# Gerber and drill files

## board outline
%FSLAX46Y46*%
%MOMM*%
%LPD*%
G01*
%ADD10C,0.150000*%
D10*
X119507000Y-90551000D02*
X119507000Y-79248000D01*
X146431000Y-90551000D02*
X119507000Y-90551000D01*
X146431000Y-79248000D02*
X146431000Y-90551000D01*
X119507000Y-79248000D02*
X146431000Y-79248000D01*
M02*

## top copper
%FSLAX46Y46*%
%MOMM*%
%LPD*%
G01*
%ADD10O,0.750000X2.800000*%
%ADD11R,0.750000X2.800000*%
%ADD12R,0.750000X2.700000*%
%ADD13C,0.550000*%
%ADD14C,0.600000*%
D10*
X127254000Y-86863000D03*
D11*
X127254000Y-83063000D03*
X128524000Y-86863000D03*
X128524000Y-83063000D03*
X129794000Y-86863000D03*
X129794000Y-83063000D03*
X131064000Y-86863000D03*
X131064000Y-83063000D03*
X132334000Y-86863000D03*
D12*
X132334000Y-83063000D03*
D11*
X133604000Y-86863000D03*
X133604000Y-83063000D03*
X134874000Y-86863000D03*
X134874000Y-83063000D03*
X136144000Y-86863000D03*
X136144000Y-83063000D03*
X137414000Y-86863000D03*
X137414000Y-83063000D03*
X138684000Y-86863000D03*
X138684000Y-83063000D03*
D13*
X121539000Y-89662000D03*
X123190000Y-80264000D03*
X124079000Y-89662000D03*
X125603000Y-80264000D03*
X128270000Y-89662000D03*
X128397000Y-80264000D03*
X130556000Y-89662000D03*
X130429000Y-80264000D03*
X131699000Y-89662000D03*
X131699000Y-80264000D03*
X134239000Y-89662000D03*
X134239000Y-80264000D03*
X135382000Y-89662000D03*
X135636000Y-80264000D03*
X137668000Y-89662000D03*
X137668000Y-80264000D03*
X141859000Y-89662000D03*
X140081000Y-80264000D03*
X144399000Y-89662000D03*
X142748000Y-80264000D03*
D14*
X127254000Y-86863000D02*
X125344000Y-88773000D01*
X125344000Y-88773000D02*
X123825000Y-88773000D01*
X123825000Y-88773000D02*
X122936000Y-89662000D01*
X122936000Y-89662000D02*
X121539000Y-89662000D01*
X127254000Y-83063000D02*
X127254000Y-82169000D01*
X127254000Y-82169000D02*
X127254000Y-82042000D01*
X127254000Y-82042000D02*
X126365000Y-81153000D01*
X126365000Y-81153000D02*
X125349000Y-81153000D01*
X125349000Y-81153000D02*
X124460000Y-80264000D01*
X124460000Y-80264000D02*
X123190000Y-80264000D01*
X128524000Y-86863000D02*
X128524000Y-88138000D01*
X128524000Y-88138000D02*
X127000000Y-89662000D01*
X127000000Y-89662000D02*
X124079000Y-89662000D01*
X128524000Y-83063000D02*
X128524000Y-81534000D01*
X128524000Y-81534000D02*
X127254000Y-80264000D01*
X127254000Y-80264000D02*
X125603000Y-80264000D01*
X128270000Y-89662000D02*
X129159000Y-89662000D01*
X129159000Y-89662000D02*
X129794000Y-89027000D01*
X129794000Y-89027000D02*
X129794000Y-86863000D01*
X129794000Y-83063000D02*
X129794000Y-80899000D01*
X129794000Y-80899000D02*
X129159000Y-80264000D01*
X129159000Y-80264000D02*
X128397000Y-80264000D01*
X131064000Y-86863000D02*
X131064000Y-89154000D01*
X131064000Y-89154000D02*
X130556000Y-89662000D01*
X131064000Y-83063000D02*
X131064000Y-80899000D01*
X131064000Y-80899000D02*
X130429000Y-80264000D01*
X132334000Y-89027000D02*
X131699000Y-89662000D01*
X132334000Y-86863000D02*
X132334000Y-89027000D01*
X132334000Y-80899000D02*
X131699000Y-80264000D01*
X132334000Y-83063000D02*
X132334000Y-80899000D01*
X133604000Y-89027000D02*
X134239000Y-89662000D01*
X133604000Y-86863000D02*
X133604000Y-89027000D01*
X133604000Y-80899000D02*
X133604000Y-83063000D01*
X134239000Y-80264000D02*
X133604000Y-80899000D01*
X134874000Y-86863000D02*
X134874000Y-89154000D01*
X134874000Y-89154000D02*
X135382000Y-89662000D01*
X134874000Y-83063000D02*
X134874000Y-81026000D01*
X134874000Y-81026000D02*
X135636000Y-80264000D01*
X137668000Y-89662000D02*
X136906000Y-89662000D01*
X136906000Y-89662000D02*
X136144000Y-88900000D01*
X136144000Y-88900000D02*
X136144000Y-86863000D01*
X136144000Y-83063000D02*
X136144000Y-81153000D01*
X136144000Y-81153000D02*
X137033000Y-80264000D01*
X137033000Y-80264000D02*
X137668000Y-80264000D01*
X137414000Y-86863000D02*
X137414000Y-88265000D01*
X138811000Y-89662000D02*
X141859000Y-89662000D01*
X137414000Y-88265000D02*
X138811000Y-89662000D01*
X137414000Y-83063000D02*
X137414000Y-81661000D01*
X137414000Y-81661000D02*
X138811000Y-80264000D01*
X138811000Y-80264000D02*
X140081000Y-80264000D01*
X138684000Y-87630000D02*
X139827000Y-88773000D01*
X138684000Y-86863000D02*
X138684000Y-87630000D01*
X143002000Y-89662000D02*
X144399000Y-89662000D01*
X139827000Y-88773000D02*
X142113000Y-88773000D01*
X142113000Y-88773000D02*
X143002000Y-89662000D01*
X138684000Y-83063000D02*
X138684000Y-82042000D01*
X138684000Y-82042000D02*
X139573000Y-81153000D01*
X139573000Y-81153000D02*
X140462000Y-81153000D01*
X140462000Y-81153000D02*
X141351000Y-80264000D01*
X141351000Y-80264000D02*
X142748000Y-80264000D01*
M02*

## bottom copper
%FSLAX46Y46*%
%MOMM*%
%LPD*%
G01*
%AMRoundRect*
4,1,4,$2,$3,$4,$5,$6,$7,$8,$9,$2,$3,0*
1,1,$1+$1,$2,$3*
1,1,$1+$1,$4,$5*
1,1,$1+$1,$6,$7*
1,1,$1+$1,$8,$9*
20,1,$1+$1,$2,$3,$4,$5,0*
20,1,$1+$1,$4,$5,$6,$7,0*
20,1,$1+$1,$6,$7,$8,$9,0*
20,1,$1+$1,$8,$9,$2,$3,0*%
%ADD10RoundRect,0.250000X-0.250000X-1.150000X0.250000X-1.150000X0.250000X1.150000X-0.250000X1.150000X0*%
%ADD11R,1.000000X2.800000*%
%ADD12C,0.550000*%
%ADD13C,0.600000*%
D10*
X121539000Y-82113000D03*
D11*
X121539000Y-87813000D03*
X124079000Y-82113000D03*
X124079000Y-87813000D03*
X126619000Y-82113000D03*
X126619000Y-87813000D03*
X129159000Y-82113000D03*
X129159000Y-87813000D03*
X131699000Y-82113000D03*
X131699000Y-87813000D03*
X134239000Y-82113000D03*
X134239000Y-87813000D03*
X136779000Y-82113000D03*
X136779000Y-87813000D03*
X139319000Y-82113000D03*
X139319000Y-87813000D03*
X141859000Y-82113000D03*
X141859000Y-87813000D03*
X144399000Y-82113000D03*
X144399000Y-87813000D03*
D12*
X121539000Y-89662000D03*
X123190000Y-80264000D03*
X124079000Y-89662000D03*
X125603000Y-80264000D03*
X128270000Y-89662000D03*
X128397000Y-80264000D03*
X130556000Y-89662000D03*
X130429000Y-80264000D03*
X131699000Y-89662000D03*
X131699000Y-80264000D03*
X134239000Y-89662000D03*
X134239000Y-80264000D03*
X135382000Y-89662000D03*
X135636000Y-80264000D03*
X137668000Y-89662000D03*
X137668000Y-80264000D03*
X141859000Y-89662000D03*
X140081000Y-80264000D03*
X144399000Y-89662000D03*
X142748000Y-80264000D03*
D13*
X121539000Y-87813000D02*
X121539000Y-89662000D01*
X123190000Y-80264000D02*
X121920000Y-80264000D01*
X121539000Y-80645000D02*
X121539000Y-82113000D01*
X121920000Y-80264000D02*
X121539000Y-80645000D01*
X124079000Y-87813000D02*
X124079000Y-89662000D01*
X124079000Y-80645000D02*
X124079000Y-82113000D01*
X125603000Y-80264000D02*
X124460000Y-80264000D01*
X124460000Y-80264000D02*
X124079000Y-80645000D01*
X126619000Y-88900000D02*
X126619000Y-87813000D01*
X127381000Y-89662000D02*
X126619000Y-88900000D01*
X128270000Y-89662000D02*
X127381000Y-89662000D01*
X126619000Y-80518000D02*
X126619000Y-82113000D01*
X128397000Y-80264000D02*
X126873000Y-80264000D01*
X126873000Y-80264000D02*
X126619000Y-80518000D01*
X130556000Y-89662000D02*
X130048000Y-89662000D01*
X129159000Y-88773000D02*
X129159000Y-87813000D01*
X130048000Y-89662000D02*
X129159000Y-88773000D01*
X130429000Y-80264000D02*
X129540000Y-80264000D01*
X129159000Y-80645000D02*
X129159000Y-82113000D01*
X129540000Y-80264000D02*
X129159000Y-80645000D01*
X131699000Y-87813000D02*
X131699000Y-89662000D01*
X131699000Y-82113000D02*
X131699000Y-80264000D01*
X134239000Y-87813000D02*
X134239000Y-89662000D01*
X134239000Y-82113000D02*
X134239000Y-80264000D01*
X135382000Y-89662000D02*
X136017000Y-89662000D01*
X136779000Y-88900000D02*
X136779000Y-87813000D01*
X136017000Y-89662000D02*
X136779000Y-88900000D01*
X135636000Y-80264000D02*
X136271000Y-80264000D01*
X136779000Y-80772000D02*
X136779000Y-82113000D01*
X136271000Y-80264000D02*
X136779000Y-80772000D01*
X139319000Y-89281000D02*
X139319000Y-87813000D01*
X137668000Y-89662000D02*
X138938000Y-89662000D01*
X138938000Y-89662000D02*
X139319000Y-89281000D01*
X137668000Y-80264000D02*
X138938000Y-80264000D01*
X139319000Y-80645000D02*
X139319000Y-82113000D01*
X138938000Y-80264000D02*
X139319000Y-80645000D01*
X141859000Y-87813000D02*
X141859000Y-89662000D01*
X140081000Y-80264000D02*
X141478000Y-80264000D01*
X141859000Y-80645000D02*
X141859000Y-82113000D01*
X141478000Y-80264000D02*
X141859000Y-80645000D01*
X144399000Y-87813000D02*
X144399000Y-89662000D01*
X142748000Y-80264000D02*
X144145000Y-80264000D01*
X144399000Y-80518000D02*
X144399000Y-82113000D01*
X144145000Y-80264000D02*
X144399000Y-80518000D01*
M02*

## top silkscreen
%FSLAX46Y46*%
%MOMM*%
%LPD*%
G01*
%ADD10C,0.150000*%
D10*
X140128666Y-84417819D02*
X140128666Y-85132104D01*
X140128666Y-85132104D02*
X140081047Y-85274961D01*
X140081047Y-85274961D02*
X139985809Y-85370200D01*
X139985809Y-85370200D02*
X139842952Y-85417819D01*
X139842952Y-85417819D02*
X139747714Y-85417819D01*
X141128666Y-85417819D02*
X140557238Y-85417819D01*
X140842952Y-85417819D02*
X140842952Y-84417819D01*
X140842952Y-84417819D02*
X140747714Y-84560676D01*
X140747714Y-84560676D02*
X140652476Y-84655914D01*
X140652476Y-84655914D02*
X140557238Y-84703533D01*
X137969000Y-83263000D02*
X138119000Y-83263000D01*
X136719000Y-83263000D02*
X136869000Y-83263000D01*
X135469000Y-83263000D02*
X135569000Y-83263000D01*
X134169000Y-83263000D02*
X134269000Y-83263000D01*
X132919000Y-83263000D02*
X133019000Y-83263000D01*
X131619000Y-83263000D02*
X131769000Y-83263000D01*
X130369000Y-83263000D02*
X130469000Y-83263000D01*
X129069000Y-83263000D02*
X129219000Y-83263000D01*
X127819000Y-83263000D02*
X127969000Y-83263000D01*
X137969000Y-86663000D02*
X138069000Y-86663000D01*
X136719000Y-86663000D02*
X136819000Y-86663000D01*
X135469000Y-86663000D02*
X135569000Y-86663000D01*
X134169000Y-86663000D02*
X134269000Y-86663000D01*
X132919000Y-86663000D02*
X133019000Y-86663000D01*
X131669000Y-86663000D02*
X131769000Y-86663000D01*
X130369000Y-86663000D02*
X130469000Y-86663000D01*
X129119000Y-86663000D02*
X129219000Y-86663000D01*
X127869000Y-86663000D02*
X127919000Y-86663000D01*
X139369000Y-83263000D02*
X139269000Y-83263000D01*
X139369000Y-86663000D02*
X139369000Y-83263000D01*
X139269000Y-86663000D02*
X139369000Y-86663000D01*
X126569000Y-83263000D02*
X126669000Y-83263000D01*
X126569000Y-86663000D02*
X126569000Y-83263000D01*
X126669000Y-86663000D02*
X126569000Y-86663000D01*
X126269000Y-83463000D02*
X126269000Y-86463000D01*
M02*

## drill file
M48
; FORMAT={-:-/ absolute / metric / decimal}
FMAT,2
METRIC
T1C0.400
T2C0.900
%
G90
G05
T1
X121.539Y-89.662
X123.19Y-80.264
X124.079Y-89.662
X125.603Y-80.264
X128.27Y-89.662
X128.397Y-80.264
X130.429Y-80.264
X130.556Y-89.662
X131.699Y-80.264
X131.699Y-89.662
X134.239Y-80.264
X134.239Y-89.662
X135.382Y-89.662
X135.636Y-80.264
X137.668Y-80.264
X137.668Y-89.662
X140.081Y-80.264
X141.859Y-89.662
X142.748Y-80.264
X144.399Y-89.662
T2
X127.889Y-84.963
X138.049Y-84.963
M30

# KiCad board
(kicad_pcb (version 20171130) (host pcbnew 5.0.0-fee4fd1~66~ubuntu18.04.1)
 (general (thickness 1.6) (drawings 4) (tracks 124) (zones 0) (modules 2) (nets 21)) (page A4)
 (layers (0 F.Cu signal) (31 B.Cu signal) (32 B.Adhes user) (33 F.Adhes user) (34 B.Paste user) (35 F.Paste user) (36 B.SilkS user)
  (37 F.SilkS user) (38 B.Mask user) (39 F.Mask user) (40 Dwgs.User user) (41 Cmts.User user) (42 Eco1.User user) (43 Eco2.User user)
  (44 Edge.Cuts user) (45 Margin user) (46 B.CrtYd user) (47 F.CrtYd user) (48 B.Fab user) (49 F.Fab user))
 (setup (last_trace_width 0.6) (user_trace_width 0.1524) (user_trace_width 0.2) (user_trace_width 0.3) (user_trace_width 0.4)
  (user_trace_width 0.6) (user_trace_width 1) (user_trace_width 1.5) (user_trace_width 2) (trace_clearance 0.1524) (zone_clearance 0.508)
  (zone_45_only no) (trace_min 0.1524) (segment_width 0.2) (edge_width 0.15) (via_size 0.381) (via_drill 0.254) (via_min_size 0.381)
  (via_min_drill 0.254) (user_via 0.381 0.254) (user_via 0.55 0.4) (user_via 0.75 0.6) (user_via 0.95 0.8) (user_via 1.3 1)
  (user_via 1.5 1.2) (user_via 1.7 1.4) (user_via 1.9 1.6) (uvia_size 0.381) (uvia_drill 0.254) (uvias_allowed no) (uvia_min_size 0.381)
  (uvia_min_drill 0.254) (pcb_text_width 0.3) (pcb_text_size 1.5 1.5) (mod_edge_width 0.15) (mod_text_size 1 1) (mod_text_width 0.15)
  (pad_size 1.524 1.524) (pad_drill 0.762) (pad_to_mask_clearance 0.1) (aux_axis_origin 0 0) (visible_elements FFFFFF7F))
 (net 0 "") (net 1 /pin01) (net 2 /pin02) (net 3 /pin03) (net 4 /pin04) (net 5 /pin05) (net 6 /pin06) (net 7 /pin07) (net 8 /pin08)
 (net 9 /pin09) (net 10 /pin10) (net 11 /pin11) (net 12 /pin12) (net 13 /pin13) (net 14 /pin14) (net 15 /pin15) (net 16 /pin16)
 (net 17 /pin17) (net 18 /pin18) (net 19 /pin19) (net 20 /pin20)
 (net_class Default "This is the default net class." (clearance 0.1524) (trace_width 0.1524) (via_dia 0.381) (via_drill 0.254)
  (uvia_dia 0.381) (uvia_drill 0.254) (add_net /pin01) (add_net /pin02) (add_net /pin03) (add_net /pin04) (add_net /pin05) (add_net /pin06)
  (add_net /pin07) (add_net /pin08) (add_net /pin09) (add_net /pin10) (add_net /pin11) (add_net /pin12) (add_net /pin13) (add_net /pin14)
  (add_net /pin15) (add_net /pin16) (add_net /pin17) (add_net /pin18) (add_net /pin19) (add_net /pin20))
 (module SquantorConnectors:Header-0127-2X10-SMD (layer F.Cu) (at 132.969 84.963)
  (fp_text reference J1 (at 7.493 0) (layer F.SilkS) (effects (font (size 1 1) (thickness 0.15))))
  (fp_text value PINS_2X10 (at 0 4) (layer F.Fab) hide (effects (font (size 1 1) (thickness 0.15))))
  (fp_line (start 5 -1.7) (end 5.15 -1.7) (layer F.SilkS) (width 0.15))
  (fp_line (start 3.75 -1.7) (end 3.9 -1.7) (layer F.SilkS) (width 0.15))
  (fp_line (start 2.5 -1.7) (end 2.6 -1.7) (layer F.SilkS) (width 0.15))
  (fp_line (start 1.2 -1.7) (end 1.3 -1.7) (layer F.SilkS) (width 0.15))
  (fp_line (start -0.05 -1.7) (end 0.05 -1.7) (layer F.SilkS) (width 0.15))
  (fp_line (start -1.35 -1.7) (end -1.2 -1.7) (layer F.SilkS) (width 0.15))
  (fp_line (start -2.6 -1.7) (end -2.5 -1.7) (layer F.SilkS) (width 0.15))
  (fp_line (start -3.9 -1.7) (end -3.75 -1.7) (layer F.SilkS) (width 0.15))
  (fp_line (start -5.15 -1.7) (end -5 -1.7) (layer F.SilkS) (width 0.15))
  (fp_line (start 5 1.7) (end 5.1 1.7) (layer F.SilkS) (width 0.15))
  (fp_line (start 3.75 1.7) (end 3.85 1.7) (layer F.SilkS) (width 0.15))
  (fp_line (start 2.5 1.7) (end 2.6 1.7) (layer F.SilkS) (width 0.15))
  (fp_line (start 1.2 1.7) (end 1.3 1.7) (layer F.SilkS) (width 0.15))
  (fp_line (start -0.05 1.7) (end 0.05 1.7) (layer F.SilkS) (width 0.15))
  (fp_line (start -1.3 1.7) (end -1.2 1.7) (layer F.SilkS) (width 0.15))
  (fp_line (start -2.6 1.7) (end -2.5 1.7) (layer F.SilkS) (width 0.15))
  (fp_line (start -3.85 1.7) (end -3.75 1.7) (layer F.SilkS) (width 0.15))
  (fp_line (start -5.1 1.7) (end -5.05 1.7) (layer F.SilkS) (width 0.15))
  (fp_line (start 6.4 -1.7) (end 6.3 -1.7) (layer F.SilkS) (width 0.15))
  (fp_line (start 6.4 1.7) (end 6.4 -1.7) (layer F.SilkS) (width 0.15))
  (fp_line (start 6.3 1.7) (end 6.4 1.7) (layer F.SilkS) (width 0.15))
  (fp_line (start -6.4 -1.7) (end -6.3 -1.7) (layer F.SilkS) (width 0.15))
  (fp_line (start -6.4 1.7) (end -6.4 -1.7) (layer F.SilkS) (width 0.15))
  (fp_line (start -6.3 1.7) (end -6.4 1.7) (layer F.SilkS) (width 0.15))
  (fp_line (start -6.7 -1.5) (end -6.7 1.5) (layer F.SilkS) (width 0.15))
  (pad 1 smd oval (at -5.715 1.9) (size 0.75 2.8) (layers F.Cu F.Paste F.Mask) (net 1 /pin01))
  (pad 2 smd rect (at -5.715 -1.9) (size 0.75 2.8) (layers F.Cu F.Paste F.Mask) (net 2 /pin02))
  (pad 3 smd rect (at -4.445 1.9) (size 0.75 2.8) (layers F.Cu F.Paste F.Mask) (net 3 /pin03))
  (pad 4 smd rect (at -4.445 -1.9) (size 0.75 2.8) (layers F.Cu F.Paste F.Mask) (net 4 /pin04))
  (pad 5 smd rect (at -3.175 1.9) (size 0.75 2.8) (layers F.Cu F.Paste F.Mask) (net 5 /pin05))
  (pad 6 smd rect (at -3.175 -1.9) (size 0.75 2.8) (layers F.Cu F.Paste F.Mask) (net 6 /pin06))
  (pad 7 smd rect (at -1.905 1.9) (size 0.75 2.8) (layers F.Cu F.Paste F.Mask) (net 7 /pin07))
  (pad 8 smd rect (at -1.905 -1.9) (size 0.75 2.8) (layers F.Cu F.Paste F.Mask) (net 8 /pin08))
  (pad 9 smd rect (at -0.635 1.9) (size 0.75 2.8) (layers F.Cu F.Paste F.Mask) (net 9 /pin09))
  (pad 10 smd rect (at -0.635 -1.9) (size 0.75 2.7) (layers F.Cu F.Paste F.Mask) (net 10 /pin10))
  (pad 11 smd rect (at 0.635 1.9) (size 0.75 2.8) (layers F.Cu F.Paste F.Mask) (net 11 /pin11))
  (pad 12 smd rect (at 0.635 -1.9) (size 0.75 2.8) (layers F.Cu F.Paste F.Mask) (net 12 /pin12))
  (pad 13 smd rect (at 1.905 1.9) (size 0.75 2.8) (layers F.Cu F.Paste F.Mask) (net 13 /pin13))
  (pad 14 smd rect (at 1.905 -1.9) (size 0.75 2.8) (layers F.Cu F.Paste F.Mask) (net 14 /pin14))
  (pad 15 smd rect (at 3.175 1.9) (size 0.75 2.8) (layers F.Cu F.Paste F.Mask) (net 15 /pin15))
  (pad 16 smd rect (at 3.175 -1.9) (size 0.75 2.8) (layers F.Cu F.Paste F.Mask) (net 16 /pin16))
  (pad 17 smd rect (at 4.445 1.9) (size 0.75 2.8) (layers F.Cu F.Paste F.Mask) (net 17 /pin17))
  (pad 18 smd rect (at 4.445 -1.9) (size 0.75 2.8) (layers F.Cu F.Paste F.Mask) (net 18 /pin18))
  (pad 19 smd rect (at 5.715 1.9) (size 0.75 2.8) (layers F.Cu F.Paste F.Mask) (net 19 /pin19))
  (pad 20 smd rect (at 5.715 -1.9) (size 0.75 2.8) (layers F.Cu F.Paste F.Mask) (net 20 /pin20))
  (pad "" np_thru_hole circle (at -5.08 0) (size 0.9 0.9) (drill 0.9) (layers *.Cu *.Mask))
  (pad "" np_thru_hole circle (at 5.08 0) (size 0.9 0.9) (drill 0.9) (layers *.Cu *.Mask)))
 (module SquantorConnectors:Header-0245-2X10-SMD (layer B.Cu) (at 132.969 84.963)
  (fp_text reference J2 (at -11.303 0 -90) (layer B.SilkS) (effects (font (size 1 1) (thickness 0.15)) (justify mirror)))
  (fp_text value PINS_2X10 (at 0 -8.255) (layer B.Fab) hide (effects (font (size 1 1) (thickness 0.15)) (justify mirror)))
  (pad 1 smd roundrect (at -11.43 -2.85) (size 1 2.8) (layers B.Cu B.Paste B.Mask) (roundrect_rratio 0.25) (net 2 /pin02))
  (pad 2 smd rect (at -11.43 2.85) (size 1 2.8) (layers B.Cu B.Paste B.Mask) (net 1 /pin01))
  (pad 3 smd rect (at -8.89 -2.85) (size 1 2.8) (layers B.Cu B.Paste B.Mask) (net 4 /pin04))
  (pad 4 smd rect (at -8.89 2.85) (size 1 2.8) (layers B.Cu B.Paste B.Mask) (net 3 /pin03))
  (pad 5 smd rect (at -6.35 -2.85) (size 1 2.8) (layers B.Cu B.Paste B.Mask) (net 6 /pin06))
  (pad 6 smd rect (at -6.35 2.85) (size 1 2.8) (layers B.Cu B.Paste B.Mask) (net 5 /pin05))
  (pad 7 smd rect (at -3.81 -2.85) (size 1 2.8) (layers B.Cu B.Paste B.Mask) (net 8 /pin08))
  (pad 8 smd rect (at -3.81 2.85) (size 1 2.8) (layers B.Cu B.Paste B.Mask) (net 7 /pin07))
  (pad 9 smd rect (at -1.27 -2.85) (size 1 2.8) (layers B.Cu B.Paste B.Mask) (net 10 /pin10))
  (pad 10 smd rect (at -1.27 2.85) (size 1 2.8) (layers B.Cu B.Paste B.Mask) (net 9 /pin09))
  (pad 11 smd rect (at 1.27 -2.85) (size 1 2.8) (layers B.Cu B.Paste B.Mask) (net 12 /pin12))
  (pad 12 smd rect (at 1.27 2.85) (size 1 2.8) (layers B.Cu B.Paste B.Mask) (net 11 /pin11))
  (pad 13 smd rect (at 3.81 -2.85) (size 1 2.8) (layers B.Cu B.Paste B.Mask) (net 14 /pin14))
  (pad 14 smd rect (at 3.81 2.85) (size 1 2.8) (layers B.Cu B.Paste B.Mask) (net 13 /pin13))
  (pad 15 smd rect (at 6.35 -2.85) (size 1 2.8) (layers B.Cu B.Paste B.Mask) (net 16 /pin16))
  (pad 16 smd rect (at 6.35 2.85) (size 1 2.8) (layers B.Cu B.Paste B.Mask) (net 15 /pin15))
  (pad 17 smd rect (at 8.89 -2.85) (size 1 2.8) (layers B.Cu B.Paste B.Mask) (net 18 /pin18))
  (pad 18 smd rect (at 8.89 2.85) (size 1 2.8) (layers B.Cu B.Paste B.Mask) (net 17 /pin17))
  (pad 19 smd rect (at 11.43 -2.85) (size 1 2.8) (layers B.Cu B.Paste B.Mask) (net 20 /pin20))
  (pad 20 smd rect (at 11.43 2.85) (size 1 2.8) (layers B.Cu B.Paste B.Mask) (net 19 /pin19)))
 (gr_line (start 119.507 90.551) (end 119.507 79.248) (layer Edge.Cuts) (width 0.15))
 (gr_line (start 146.431 90.551) (end 119.507 90.551) (layer Edge.Cuts) (width 0.15))
 (gr_line (start 146.431 79.248) (end 146.431 90.551) (layer Edge.Cuts) (width 0.15))
 (gr_line (start 119.507 79.248) (end 146.431 79.248) (layer Edge.Cuts) (width 0.15))
 (segment (start 127.254 86.863) (end 125.344 88.773) (width 0.6) (layer F.Cu) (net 1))
 (segment (start 125.344 88.773) (end 123.825 88.773) (width 0.6) (layer F.Cu) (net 1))
 (segment (start 123.825 88.773) (end 122.936 89.662) (width 0.6) (layer F.Cu) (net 1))
 (via (at 121.539 89.662) (size 0.55) (drill 0.4) (layers F.Cu B.Cu) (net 1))
 (segment (start 122.936 89.662) (end 121.539 89.662) (width 0.6) (layer F.Cu) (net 1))
 (segment (start 121.539 87.813) (end 121.539 89.662) (width 0.6) (layer B.Cu) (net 1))
 (segment (start 127.254 83.063) (end 127.254 82.169) (width 0.6) (layer F.Cu) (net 2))
 (segment (start 127.254 82.169) (end 127.254 82.042) (width 0.6) (layer F.Cu) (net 2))
 (segment (start 127.254 82.042) (end 126.365 81.153) (width 0.6) (layer F.Cu) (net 2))
 (segment (start 126.365 81.153) (end 125.349 81.153) (width 0.6) (layer F.Cu) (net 2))
 (segment (start 125.349 81.153) (end 124.46 80.264) (width 0.6) (layer F.Cu) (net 2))
 (via (at 123.19 80.264) (size 0.55) (drill 0.4) (layers F.Cu B.Cu) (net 2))
 (segment (start 124.46 80.264) (end 123.19 80.264) (width 0.6) (layer F.Cu) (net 2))
 (segment (start 123.19 80.264) (end 121.92 80.264) (width 0.6) (layer B.Cu) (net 2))
 (segment (start 121.539 80.645) (end 121.539 82.113) (width 0.6) (layer B.Cu) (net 2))
 (segment (start 121.92 80.264) (end 121.539 80.645) (width 0.6) (layer B.Cu) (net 2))
 (segment (start 128.524 86.863) (end 128.524 88.138) (width 0.6) (layer F.Cu) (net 3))
 (segment (start 128.524 88.138) (end 127 89.662) (width 0.6) (layer F.Cu) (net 3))
 (via (at 124.079 89.662) (size 0.55) (drill 0.4) (layers F.Cu B.Cu) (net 3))
 (segment (start 127 89.662) (end 124.079 89.662) (width 0.6) (layer F.Cu) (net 3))
 (segment (start 124.079 87.813) (end 124.079 89.662) (width 0.6) (layer B.Cu) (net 3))
 (segment (start 128.524 83.063) (end 128.524 81.534) (width 0.6) (layer F.Cu) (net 4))
 (segment (start 128.524 81.534) (end 127.254 80.264) (width 0.6) (layer F.Cu) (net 4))
 (via (at 125.603 80.264) (size 0.55) (drill 0.4) (layers F.Cu B.Cu) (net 4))
 (segment (start 127.254 80.264) (end 125.603 80.264) (width 0.6) (layer F.Cu) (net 4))
 (segment (start 124.079 80.645) (end 124.079 82.113) (width 0.6) (layer B.Cu) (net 4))
 (segment (start 125.603 80.264) (end 124.46 80.264) (width 0.6) (layer B.Cu) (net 4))
 (segment (start 124.46 80.264) (end 124.079 80.645) (width 0.6) (layer B.Cu) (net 4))
 (segment (start 126.619 88.9) (end 126.619 87.813) (width 0.6) (layer B.Cu) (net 5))
 (segment (start 128.27 89.662) (end 129.159 89.662) (width 0.6) (layer F.Cu) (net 5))
 (segment (start 129.159 89.662) (end 129.794 89.027) (width 0.6) (layer F.Cu) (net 5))
 (via (at 128.27 89.662) (size 0.55) (drill 0.4) (layers F.Cu B.Cu) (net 5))
 (segment (start 129.794 89.027) (end 129.794 86.863) (width 0.6) (layer F.Cu) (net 5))
 (segment (start 127.381 89.662) (end 126.619 88.9) (width 0.6) (layer B.Cu) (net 5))
 (segment (start 128.27 89.662) (end 127.381 89.662) (width 0.6) (layer B.Cu) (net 5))
 (segment (start 129.794 83.063) (end 129.794 80.899) (width 0.6) (layer F.Cu) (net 6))
 (via (at 128.397 80.264) (size 0.55) (drill 0.4) (layers F.Cu B.Cu) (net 6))
 (segment (start 129.794 80.899) (end 129.159 80.264) (width 0.6) (layer F.Cu) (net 6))
 (segment (start 129.159 80.264) (end 128.397 80.264) (width 0.6) (layer F.Cu) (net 6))
 (segment (start 126.619 80.518) (end 126.619 82.113) (width 0.6) (layer B.Cu) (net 6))
 (segment (start 128.397 80.264) (end 126.873 80.264) (width 0.6) (layer B.Cu) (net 6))
 (segment (start 126.873 80.264) (end 126.619 80.518) (width 0.6) (layer B.Cu) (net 6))
 (segment (start 131.064 86.863) (end 131.064 89.154) (width 0.6) (layer F.Cu) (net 7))
 (via (at 130.556 89.662) (size 0.55) (drill 0.4) (layers F.Cu B.Cu) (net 7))
 (segment (start 131.064 89.154) (end 130.556 89.662) (width 0.6) (layer F.Cu) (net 7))
 (segment (start 130.556 89.662) (end 130.048 89.662) (width 0.6) (layer B.Cu) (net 7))
 (segment (start 129.159 88.773) (end 129.159 87.813) (width 0.6) (layer B.Cu) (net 7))
 (segment (start 130.048 89.662) (end 129.159 88.773) (width 0.6) (layer B.Cu) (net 7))
 (segment (start 131.064 83.063) (end 131.064 80.899) (width 0.6) (layer F.Cu) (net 8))
 (via (at 130.429 80.264) (size 0.55) (drill 0.4) (layers F.Cu B.Cu) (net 8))
 (segment (start 131.064 80.899) (end 130.429 80.264) (width 0.6) (layer F.Cu) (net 8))
 (segment (start 130.429 80.264) (end 129.54 80.264) (width 0.6) (layer B.Cu) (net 8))
 (segment (start 129.159 80.645) (end 129.159 82.113) (width 0.6) (layer B.Cu) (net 8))
 (segment (start 129.54 80.264) (end 129.159 80.645) (width 0.6) (layer B.Cu) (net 8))
 (via (at 131.699 89.662) (size 0.55) (drill 0.4) (layers F.Cu B.Cu) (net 9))
 (segment (start 131.699 87.813) (end 131.699 89.662) (width 0.6) (layer B.Cu) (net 9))
 (segment (start 132.334 89.027) (end 131.699 89.662) (width 0.6) (layer F.Cu) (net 9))
 (segment (start 132.334 86.863) (end 132.334 89.027) (width 0.6) (layer F.Cu) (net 9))
 (via (at 131.699 80.264) (size 0.55) (drill 0.4) (layers F.Cu B.Cu) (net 10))
 (segment (start 131.699 82.113) (end 131.699 80.264) (width 0.6) (layer B.Cu) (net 10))
 (segment (start 132.334 80.899) (end 131.699 80.264) (width 0.6) (layer F.Cu) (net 10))
 (segment (start 132.334 83.063) (end 132.334 80.899) (width 0.6) (layer F.Cu) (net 10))
 (via (at 134.239 89.662) (size 0.55) (drill 0.4) (layers F.Cu B.Cu) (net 11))
 (segment (start 134.239 87.813) (end 134.239 89.662) (width 0.6) (layer B.Cu) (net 11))
 (segment (start 133.604 89.027) (end 134.239 89.662) (width 0.6) (layer F.Cu) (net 11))
 (segment (start 133.604 86.863) (end 133.604 89.027) (width 0.6) (layer F.Cu) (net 11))
 (via (at 134.239 80.264) (size 0.55) (drill 0.4) (layers F.Cu B.Cu) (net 12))
 (segment (start 134.239 82.113) (end 134.239 80.264) (width 0.6) (layer B.Cu) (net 12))
 (segment (start 133.604 80.899) (end 133.604 83.063) (width 0.6) (layer F.Cu) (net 12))
 (segment (start 134.239 80.264) (end 133.604 80.899) (width 0.6) (layer F.Cu) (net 12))
 (segment (start 134.874 86.863) (end 134.874 89.154) (width 0.6) (layer F.Cu) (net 13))
 (via (at 135.382 89.662) (size 0.55) (drill 0.4) (layers F.Cu B.Cu) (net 13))
 (segment (start 134.874 89.154) (end 135.382 89.662) (width 0.6) (layer F.Cu) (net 13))
 (segment (start 135.382 89.662) (end 136.017 89.662) (width 0.6) (layer B.Cu) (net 13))
 (segment (start 136.779 88.9) (end 136.779 87.813) (width 0.6) (layer B.Cu) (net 13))
 (segment (start 136.017 89.662) (end 136.779 88.9) (width 0.6) (layer B.Cu) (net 13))
 (segment (start 134.874 83.063) (end 134.874 81.026) (width 0.6) (layer F.Cu) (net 14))
 (via (at 135.636 80.264) (size 0.55) (drill 0.4) (layers F.Cu B.Cu) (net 14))
 (segment (start 134.874 81.026) (end 135.636 80.264) (width 0.6) (layer F.Cu) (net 14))
 (segment (start 135.636 80.264) (end 136.271 80.264) (width 0.6) (layer B.Cu) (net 14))
 (segment (start 136.779 80.772) (end 136.779 82.113) (width 0.6) (layer B.Cu) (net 14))
 (segment (start 136.271 80.264) (end 136.779 80.772) (width 0.6) (layer B.Cu) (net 14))
 (segment (start 139.319 89.281) (end 139.319 87.813) (width 0.6) (layer B.Cu) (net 15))
 (segment (start 137.668 89.662) (end 136.906 89.662) (width 0.6) (layer F.Cu) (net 15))
 (segment (start 136.906 89.662) (end 136.144 88.9) (width 0.6) (layer F.Cu) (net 15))
 (via (at 137.668 89.662) (size 0.55) (drill 0.4) (layers F.Cu B.Cu) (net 15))
 (segment (start 136.144 88.9) (end 136.144 86.863) (width 0.6) (layer F.Cu) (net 15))
 (segment (start 137.668 89.662) (end 138.938 89.662) (width 0.6) (layer B.Cu) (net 15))
 (segment (start 138.938 89.662) (end 139.319 89.281) (width 0.6) (layer B.Cu) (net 15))
 (segment (start 136.144 83.063) (end 136.144 81.153) (width 0.6) (layer F.Cu) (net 16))
 (via (at 137.668 80.264) (size 0.55) (drill 0.4) (layers F.Cu B.Cu) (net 16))
 (segment (start 136.144 81.153) (end 137.033 80.264) (width 0.6) (layer F.Cu) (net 16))
 (segment (start 137.033 80.264) (end 137.668 80.264) (width 0.6) (layer F.Cu) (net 16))
 (segment (start 137.668 80.264) (end 138.938 80.264) (width 0.6) (layer B.Cu) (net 16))
 (segment (start 139.319 80.645) (end 139.319 82.113) (width 0.6) (layer B.Cu) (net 16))
 (segment (start 138.938 80.264) (end 139.319 80.645) (width 0.6) (layer B.Cu) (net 16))
 (via (at 141.859 89.662) (size 0.55) (drill 0.4) (layers F.Cu B.Cu) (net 17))
 (segment (start 141.859 87.813) (end 141.859 89.662) (width 0.6) (layer B.Cu) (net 17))
 (segment (start 137.414 86.863) (end 137.414 88.265) (width 0.6) (layer F.Cu) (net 17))
 (segment (start 138.811 89.662) (end 141.859 89.662) (width 0.6) (layer F.Cu) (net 17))
 (segment (start 137.414 88.265) (end 138.811 89.662) (width 0.6) (layer F.Cu) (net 17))
 (segment (start 137.414 83.063) (end 137.414 81.661) (width 0.6) (layer F.Cu) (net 18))
 (segment (start 137.414 81.661) (end 138.811 80.264) (width 0.6) (layer F.Cu) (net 18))
 (via (at 140.081 80.264) (size 0.55) (drill 0.4) (layers F.Cu B.Cu) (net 18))
 (segment (start 138.811 80.264) (end 140.081 80.264) (width 0.6) (layer F.Cu) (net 18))
 (segment (start 140.081 80.264) (end 141.478 80.264) (width 0.6) (layer B.Cu) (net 18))
 (segment (start 141.859 80.645) (end 141.859 82.113) (width 0.6) (layer B.Cu) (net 18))
 (segment (start 141.478 80.264) (end 141.859 80.645) (width 0.6) (layer B.Cu) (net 18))
 (via (at 144.399 89.662) (size 0.55) (drill 0.4) (layers F.Cu B.Cu) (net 19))
 (segment (start 144.399 87.813) (end 144.399 89.662) (width 0.6) (layer B.Cu) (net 19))
 (segment (start 138.684 87.63) (end 139.827 88.773) (width 0.6) (layer F.Cu) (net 19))
 (segment (start 138.684 86.863) (end 138.684 87.63) (width 0.6) (layer F.Cu) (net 19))
 (segment (start 143.002 89.662) (end 144.399 89.662) (width 0.6) (layer F.Cu) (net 19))
 (segment (start 139.827 88.773) (end 142.113 88.773) (width 0.6) (layer F.Cu) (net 19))
 (segment (start 142.113 88.773) (end 143.002 89.662) (width 0.6) (layer F.Cu) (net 19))
 (segment (start 138.684 83.063) (end 138.684 82.042) (width 0.6) (layer F.Cu) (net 20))
 (segment (start 138.684 82.042) (end 139.573 81.153) (width 0.6) (layer F.Cu) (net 20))
 (segment (start 139.573 81.153) (end 140.462 81.153) (width 0.6) (layer F.Cu) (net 20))
 (via (at 142.748 80.264) (size 0.55) (drill 0.4) (layers F.Cu B.Cu) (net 20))
 (segment (start 140.462 81.153) (end 141.351 80.264) (width 0.6) (layer F.Cu) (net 20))
 (segment (start 141.351 80.264) (end 142.748 80.264) (width 0.6) (layer F.Cu) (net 20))
 (segment (start 142.748 80.264) (end 144.145 80.264) (width 0.6) (layer B.Cu) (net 20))
 (segment (start 144.399 80.518) (end 144.399 82.113) (width 0.6) (layer B.Cu) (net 20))
 (segment (start 144.145 80.264) (end 144.399 80.518) (width 0.6) (layer B.Cu) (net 20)))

